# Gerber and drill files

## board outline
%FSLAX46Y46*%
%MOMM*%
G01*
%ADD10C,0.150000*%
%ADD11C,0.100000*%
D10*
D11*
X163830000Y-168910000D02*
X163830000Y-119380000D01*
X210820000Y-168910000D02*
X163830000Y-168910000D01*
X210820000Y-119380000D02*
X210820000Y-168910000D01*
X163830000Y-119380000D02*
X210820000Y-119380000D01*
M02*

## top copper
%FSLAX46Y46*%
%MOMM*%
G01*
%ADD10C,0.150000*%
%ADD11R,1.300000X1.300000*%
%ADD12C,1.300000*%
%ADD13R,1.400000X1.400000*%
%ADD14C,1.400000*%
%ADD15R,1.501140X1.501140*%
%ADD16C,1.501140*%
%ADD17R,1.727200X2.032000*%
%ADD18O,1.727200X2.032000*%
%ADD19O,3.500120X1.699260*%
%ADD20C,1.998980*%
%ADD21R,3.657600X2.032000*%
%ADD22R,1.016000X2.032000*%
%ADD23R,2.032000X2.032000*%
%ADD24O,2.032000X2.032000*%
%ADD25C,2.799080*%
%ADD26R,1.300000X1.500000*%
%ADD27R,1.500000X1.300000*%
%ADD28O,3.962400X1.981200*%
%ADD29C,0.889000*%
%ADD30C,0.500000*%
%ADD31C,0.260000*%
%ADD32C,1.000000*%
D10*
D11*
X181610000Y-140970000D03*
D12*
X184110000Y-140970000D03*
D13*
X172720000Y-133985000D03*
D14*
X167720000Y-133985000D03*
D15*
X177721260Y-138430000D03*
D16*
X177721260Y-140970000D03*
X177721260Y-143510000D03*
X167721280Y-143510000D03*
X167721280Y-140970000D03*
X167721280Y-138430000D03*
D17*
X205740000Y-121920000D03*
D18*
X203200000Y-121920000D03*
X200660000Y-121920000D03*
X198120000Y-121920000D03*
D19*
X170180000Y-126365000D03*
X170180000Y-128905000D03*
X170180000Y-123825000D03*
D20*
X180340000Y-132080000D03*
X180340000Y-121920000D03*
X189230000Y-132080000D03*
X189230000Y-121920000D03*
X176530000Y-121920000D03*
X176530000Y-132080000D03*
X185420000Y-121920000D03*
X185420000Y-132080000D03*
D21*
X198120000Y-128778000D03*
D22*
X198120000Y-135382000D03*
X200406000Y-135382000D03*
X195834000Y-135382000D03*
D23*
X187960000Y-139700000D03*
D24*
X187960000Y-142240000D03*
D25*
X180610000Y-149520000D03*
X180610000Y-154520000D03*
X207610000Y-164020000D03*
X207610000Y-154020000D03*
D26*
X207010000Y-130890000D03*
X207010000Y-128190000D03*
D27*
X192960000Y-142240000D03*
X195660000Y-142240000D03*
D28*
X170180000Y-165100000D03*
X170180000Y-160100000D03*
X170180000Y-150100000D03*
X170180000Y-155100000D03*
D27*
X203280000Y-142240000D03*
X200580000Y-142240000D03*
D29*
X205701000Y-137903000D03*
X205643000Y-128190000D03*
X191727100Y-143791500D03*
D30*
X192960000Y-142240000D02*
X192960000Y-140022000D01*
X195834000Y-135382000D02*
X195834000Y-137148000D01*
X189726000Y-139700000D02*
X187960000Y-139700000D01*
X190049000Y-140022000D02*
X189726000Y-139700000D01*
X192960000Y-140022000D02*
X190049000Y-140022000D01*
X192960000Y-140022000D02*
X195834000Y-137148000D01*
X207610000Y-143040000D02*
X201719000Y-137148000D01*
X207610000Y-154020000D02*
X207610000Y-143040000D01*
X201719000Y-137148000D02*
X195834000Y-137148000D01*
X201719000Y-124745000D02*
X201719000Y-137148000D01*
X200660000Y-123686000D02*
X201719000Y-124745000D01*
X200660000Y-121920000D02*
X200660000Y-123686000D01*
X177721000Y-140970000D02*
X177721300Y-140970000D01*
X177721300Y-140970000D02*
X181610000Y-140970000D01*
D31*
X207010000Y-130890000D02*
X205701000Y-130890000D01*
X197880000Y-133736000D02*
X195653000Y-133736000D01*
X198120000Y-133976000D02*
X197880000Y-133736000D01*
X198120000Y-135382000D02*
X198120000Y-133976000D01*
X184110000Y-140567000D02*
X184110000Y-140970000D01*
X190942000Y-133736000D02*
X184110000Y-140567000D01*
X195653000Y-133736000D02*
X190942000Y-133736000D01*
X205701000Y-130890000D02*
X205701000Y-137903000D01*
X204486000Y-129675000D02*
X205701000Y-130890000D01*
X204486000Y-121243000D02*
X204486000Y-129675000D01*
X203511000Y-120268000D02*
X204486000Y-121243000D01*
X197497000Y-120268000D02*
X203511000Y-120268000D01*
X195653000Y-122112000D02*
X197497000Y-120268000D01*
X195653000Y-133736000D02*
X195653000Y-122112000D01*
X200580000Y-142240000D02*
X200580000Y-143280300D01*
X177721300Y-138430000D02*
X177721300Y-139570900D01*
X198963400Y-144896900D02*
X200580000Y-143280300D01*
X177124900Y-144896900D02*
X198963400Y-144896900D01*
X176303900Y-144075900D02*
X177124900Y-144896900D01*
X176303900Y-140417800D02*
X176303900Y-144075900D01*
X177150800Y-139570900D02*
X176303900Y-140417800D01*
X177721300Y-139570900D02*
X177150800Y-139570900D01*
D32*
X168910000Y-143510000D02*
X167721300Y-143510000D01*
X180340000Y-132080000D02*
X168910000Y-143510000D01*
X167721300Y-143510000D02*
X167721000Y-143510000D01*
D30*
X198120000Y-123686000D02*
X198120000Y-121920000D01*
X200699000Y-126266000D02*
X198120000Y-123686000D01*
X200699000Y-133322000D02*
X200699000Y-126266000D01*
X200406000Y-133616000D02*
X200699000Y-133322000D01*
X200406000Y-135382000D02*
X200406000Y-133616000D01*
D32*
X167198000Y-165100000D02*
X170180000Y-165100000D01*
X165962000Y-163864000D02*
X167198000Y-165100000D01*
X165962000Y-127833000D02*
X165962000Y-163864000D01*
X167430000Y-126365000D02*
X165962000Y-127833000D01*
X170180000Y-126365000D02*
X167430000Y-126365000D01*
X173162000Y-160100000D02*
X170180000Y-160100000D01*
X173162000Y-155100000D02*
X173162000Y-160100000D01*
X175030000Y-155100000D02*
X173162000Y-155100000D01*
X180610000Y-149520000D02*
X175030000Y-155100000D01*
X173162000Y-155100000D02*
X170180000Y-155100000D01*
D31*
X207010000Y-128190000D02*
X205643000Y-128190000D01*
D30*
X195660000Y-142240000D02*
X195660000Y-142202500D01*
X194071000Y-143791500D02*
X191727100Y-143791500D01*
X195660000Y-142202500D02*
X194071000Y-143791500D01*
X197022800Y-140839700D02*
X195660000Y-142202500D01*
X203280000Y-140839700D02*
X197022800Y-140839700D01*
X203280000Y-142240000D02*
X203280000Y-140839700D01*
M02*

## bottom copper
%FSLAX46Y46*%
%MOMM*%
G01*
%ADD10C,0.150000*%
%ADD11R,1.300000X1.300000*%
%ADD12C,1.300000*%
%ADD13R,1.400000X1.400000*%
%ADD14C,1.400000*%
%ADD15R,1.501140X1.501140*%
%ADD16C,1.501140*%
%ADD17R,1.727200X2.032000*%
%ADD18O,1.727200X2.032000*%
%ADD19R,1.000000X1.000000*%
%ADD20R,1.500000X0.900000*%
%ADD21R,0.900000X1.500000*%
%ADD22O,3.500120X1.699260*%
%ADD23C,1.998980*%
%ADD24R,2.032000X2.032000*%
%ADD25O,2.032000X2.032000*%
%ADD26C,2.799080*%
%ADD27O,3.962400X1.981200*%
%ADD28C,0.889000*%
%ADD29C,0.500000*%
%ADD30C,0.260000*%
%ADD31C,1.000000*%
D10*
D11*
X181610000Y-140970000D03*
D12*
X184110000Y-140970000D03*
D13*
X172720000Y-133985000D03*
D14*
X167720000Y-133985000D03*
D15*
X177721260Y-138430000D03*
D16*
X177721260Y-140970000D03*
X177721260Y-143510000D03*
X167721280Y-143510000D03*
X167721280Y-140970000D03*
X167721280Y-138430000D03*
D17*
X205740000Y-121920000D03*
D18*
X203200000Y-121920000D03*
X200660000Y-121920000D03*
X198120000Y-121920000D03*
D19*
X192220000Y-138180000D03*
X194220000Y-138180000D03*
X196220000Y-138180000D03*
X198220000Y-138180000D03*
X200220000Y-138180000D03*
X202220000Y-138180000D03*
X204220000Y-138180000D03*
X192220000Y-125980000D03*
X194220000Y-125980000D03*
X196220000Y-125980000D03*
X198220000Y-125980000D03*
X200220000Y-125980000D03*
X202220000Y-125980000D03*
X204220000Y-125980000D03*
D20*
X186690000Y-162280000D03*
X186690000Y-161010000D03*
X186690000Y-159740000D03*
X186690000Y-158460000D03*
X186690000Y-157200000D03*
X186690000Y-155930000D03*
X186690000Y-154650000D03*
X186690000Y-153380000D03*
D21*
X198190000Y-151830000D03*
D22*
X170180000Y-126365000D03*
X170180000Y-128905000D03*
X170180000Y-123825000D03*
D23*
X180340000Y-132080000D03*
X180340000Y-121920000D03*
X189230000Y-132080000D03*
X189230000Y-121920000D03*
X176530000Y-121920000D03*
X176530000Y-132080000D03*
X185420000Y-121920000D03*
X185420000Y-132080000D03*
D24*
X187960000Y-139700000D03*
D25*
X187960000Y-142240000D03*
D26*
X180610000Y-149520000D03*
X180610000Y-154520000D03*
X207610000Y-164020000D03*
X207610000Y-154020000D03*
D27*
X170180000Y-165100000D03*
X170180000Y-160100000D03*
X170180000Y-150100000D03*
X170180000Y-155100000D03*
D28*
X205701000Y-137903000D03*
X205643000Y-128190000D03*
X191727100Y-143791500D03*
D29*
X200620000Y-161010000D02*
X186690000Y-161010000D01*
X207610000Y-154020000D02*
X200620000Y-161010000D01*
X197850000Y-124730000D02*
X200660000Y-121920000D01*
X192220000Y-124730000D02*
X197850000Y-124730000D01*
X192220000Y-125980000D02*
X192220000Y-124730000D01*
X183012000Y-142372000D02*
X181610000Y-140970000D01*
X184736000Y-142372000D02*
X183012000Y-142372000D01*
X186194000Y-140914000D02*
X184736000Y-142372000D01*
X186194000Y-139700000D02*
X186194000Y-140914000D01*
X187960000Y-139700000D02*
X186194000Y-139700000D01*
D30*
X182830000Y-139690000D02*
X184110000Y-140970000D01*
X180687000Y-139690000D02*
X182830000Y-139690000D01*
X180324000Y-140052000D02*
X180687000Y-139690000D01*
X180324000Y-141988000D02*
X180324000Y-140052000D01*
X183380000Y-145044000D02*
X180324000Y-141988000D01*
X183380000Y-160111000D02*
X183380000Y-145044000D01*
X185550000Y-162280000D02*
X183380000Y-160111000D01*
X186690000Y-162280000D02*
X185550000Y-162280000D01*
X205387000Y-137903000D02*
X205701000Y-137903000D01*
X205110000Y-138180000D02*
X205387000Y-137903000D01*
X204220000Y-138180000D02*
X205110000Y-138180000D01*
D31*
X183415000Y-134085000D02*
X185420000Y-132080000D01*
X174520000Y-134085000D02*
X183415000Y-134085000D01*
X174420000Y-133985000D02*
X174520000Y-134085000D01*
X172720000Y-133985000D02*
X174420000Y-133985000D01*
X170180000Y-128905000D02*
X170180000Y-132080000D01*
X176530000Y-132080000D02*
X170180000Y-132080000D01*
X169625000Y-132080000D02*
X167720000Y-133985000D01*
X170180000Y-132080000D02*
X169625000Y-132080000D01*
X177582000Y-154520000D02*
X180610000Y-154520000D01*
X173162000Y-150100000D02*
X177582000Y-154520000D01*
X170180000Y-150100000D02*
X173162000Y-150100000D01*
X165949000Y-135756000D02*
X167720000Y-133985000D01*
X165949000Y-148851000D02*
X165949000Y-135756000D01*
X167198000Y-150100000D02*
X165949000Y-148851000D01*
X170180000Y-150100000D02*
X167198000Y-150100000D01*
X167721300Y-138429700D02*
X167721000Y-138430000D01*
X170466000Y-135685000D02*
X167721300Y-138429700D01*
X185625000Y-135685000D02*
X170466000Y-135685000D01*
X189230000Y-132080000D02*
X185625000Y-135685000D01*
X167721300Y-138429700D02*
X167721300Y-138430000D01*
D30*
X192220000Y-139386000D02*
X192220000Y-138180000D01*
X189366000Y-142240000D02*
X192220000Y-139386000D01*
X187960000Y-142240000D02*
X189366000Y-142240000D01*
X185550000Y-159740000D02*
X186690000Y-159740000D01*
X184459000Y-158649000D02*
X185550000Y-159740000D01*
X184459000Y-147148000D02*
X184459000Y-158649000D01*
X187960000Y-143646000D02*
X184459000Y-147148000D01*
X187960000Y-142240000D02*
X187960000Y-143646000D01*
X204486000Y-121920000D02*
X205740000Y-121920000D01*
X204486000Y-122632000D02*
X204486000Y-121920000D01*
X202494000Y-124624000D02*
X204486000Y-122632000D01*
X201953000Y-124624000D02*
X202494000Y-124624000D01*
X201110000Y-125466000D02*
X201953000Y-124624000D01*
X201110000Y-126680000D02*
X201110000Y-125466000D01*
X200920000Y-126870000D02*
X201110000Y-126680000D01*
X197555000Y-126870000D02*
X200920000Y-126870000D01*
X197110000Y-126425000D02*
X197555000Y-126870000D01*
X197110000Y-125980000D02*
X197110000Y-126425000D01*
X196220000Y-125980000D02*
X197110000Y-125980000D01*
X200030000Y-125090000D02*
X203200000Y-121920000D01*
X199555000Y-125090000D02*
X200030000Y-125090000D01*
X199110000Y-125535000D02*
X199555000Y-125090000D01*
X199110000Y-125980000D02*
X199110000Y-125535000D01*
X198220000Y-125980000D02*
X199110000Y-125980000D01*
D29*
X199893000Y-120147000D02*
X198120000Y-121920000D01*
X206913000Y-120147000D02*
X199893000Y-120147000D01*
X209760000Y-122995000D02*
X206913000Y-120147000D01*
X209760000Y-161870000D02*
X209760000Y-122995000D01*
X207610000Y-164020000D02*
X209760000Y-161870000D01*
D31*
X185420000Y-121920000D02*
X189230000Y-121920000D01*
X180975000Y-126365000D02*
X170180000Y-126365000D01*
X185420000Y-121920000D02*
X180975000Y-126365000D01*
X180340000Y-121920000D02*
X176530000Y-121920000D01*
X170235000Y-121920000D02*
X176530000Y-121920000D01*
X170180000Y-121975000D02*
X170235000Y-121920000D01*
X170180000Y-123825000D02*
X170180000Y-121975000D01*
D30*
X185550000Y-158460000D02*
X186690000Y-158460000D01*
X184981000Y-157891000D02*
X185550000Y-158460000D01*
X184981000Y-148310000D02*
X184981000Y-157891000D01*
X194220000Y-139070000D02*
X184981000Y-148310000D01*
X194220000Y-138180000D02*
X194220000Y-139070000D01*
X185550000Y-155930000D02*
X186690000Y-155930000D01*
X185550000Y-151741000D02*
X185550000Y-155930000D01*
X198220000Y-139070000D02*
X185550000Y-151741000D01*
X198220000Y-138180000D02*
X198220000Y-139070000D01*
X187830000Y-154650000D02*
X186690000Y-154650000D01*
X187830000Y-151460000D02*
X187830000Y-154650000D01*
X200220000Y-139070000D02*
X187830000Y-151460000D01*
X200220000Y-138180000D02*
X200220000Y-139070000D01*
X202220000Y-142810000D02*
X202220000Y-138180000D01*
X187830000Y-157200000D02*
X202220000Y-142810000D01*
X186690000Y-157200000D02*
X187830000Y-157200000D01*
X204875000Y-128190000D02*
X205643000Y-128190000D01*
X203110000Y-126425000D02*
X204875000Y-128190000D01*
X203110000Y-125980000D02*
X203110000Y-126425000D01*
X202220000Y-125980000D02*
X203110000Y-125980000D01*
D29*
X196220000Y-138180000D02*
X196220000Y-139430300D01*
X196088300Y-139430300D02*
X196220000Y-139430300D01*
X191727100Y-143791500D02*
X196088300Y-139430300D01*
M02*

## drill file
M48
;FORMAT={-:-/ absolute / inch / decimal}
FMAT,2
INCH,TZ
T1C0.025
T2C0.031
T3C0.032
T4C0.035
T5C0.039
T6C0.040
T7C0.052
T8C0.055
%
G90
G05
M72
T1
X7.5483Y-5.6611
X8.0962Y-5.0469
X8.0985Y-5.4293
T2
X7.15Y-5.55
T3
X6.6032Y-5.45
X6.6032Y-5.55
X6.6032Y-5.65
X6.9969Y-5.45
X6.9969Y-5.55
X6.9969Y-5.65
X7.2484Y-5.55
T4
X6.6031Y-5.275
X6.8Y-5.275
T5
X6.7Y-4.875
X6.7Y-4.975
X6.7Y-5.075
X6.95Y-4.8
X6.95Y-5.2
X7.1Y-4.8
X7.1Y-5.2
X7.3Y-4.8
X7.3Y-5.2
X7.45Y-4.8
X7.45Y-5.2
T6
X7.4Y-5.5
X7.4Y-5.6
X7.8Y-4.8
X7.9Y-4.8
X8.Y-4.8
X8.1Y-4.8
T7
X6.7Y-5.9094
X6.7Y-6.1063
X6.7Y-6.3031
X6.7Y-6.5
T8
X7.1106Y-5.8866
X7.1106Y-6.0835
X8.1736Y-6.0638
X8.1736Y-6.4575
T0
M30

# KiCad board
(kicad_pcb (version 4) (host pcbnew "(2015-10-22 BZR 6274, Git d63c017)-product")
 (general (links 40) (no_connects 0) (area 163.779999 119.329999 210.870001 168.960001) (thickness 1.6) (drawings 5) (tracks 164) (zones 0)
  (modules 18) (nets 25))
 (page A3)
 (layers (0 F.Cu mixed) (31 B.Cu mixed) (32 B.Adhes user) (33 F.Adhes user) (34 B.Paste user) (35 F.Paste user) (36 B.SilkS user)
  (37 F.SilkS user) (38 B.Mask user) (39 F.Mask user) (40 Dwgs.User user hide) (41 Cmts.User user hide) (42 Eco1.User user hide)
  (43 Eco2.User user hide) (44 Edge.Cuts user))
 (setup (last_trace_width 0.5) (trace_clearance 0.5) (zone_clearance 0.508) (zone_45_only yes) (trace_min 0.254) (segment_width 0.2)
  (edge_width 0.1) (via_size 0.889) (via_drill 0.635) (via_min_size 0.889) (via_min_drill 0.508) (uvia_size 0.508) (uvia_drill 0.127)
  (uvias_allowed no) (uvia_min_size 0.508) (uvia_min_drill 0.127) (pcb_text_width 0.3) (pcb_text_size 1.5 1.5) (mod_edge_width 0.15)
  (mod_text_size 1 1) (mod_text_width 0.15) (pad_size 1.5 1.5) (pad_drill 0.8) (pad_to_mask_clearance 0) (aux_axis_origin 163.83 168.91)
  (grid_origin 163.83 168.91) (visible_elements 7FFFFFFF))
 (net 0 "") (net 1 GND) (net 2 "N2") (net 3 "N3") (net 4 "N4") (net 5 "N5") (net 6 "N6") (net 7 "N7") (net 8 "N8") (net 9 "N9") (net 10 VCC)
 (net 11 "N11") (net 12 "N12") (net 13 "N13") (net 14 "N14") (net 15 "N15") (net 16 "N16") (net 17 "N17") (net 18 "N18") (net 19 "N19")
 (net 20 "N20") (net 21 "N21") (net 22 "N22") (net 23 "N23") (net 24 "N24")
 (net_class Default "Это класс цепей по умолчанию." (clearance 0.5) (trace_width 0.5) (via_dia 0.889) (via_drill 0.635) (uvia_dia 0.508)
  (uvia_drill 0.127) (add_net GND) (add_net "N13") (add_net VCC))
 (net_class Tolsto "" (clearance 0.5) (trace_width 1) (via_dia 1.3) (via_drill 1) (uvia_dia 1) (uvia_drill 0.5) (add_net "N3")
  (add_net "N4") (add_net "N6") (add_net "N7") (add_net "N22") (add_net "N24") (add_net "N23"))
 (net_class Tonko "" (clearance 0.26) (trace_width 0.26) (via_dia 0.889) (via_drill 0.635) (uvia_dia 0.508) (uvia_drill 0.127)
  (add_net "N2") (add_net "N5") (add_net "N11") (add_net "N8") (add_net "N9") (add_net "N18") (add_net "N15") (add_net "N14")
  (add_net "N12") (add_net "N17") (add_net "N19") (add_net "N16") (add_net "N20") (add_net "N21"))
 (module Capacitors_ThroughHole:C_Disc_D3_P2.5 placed (layer F.Cu) (at 181.61 140.97)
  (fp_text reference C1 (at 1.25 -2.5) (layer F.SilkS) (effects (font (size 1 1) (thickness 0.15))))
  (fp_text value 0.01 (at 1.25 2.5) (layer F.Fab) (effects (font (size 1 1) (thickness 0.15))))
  (pad 1 thru_hole rect (at 0 0) (size 1.3 1.3) (drill 0.8) (layers *.Cu *.Mask F.SilkS) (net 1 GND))
  (pad 2 thru_hole circle (at 2.5 0) (size 1.3 1.3) (drill 0.8001) (layers *.Cu *.Mask F.SilkS) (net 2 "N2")))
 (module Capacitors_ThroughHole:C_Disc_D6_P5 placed (layer F.Cu) (at 172.72 133.985 180)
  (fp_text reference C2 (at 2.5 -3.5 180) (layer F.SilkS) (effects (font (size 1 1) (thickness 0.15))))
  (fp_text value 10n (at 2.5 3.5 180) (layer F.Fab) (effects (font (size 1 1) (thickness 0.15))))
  (pad 1 thru_hole rect (at 0 0 180) (size 1.4 1.4) (drill 0.9) (layers *.Cu *.Mask F.SilkS) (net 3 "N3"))
  (pad 2 thru_hole circle (at 5 0 180) (size 1.4 1.4) (drill 0.9) (layers *.Cu *.Mask F.SilkS) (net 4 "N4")))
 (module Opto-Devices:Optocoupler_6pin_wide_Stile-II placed (layer B.Cu) (at 172.72 140.97 270)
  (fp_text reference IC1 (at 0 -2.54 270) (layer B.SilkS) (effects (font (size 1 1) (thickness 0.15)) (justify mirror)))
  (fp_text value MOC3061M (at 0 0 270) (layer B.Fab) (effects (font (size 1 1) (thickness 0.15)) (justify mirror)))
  (pad 1 thru_hole rect (at -2.54 -5.00126 270) (size 1.50114 1.50114) (drill 0.8001) (layers *.Cu *.Mask B.SilkS) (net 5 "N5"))
  (pad 2 thru_hole circle (at 0 -5.00126 270) (size 1.50114 1.50114) (drill 0.8001) (layers *.Cu *.Mask B.SilkS) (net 1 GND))
  (pad 3 thru_hole circle (at 2.54 -5.00126 270) (size 1.50114 1.50114) (drill 0.8001) (layers *.Cu *.Mask B.SilkS))
  (pad 4 thru_hole circle (at 2.54 4.99872 270) (size 1.50114 1.50114) (drill 0.8001) (layers *.Cu *.Mask B.SilkS) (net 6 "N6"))
  (pad 5 thru_hole circle (at 0 4.99872 270) (size 1.50114 1.50114) (drill 0.8001) (layers *.Cu *.Mask B.SilkS))
  (pad 6 thru_hole circle (at -2.54 4.99872 270) (size 1.50114 1.50114) (drill 0.8001) (layers *.Cu *.Mask B.SilkS) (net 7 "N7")))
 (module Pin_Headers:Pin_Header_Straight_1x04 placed (layer F.Cu) (at 205.74 121.92 270)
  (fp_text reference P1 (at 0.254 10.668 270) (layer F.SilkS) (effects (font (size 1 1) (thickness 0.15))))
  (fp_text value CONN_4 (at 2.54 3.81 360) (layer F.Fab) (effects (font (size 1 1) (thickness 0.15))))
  (pad 1 thru_hole rect (at 0 0 270) (size 2.032 1.7272) (drill 1.016) (layers *.Cu *.Mask F.SilkS) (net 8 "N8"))
  (pad 2 thru_hole oval (at 0 2.54 270) (size 2.032 1.7272) (drill 1.016) (layers *.Cu *.Mask F.SilkS) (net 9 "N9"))
  (pad 3 thru_hole oval (at 0 5.08 270) (size 2.032 1.7272) (drill 1.016) (layers *.Cu *.Mask F.SilkS) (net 1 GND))
  (pad 4 thru_hole oval (at 0 7.62 270) (size 2.032 1.7272) (drill 1.016) (layers *.Cu *.Mask F.SilkS) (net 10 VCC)))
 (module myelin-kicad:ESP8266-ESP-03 (layer B.Cu) (at 198.12 132.08 90)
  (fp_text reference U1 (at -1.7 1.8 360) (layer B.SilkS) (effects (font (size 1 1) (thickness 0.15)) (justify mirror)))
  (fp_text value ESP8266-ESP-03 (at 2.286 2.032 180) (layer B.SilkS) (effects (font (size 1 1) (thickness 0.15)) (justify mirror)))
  (pad 14 smd rect (at -6.1 -5.9 90) (size 1 1) (layers B.Cu B.Paste B.Mask) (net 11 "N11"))
  (pad 13 smd rect (at -6.1 -3.9 90) (size 1 1) (layers B.Cu B.Paste B.Mask) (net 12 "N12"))
  (pad 12 smd rect (at -6.1 -1.9 90) (size 1 1) (layers B.Cu B.Paste B.Mask) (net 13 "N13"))
  (pad 11 smd rect (at -6.1 0.1 90) (size 1 1) (layers B.Cu B.Paste B.Mask) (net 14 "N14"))
  (pad 10 smd rect (at -6.1 2.1 90) (size 1 1) (layers B.Cu B.Paste B.Mask) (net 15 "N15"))
  (pad 9 smd rect (at -6.1 4.1 90) (size 1 1) (layers B.Cu B.Paste B.Mask) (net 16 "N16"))
  (pad 8 smd rect (at -6.1 6.1 90) (size 1 1) (layers B.Cu B.Paste B.Mask) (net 2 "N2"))
  (pad 1 smd rect (at 6.1 -5.9 90) (size 1 1) (layers B.Cu B.Paste B.Mask) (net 1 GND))
  (pad 2 smd rect (at 6.1 -3.9 90) (size 1 1) (layers B.Cu B.Paste B.Mask))
  (pad 3 smd rect (at 6.1 -1.9 90) (size 1 1) (layers B.Cu B.Paste B.Mask) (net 8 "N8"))
  (pad 4 smd rect (at 6.1 0.1 90) (size 1 1) (layers B.Cu B.Paste B.Mask) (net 9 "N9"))
  (pad 5 smd rect (at 6.1 2.1 90) (size 1 1) (layers B.Cu B.Paste B.Mask) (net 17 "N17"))
  (pad 6 smd rect (at 6.1 4.1 90) (size 1 1) (layers B.Cu B.Paste B.Mask) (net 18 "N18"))
  (pad 7 smd rect (at 6.1 6.1 90) (size 1 1) (layers B.Cu B.Paste B.Mask) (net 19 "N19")))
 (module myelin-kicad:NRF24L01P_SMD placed (layer B.Cu) (at 186.69 163.83)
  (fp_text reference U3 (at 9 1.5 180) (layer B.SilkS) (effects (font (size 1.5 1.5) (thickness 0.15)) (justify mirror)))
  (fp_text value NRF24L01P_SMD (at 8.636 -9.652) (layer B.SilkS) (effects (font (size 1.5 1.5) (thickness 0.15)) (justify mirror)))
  (pad 1 smd rect (at 0 -1.55) (size 1.5 0.9) (layers B.Cu B.Paste B.Mask) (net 2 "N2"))
  (pad 2 smd rect (at 0 -2.82) (size 1.5 0.9) (layers B.Cu B.Paste B.Mask) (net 1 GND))
  (pad 3 smd rect (at 0 -4.09) (size 1.5 0.9) (layers B.Cu B.Paste B.Mask) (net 11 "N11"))
  (pad 4 smd rect (at 0 -5.37) (size 1.5 0.9) (layers B.Cu B.Paste B.Mask) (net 12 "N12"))
  (pad 5 smd rect (at 0 -6.63) (size 1.5 0.9) (layers B.Cu B.Paste B.Mask) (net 16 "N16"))
  (pad 6 smd rect (at 0 -7.9) (size 1.5 0.9) (layers B.Cu B.Paste B.Mask) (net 14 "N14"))
  (pad 7 smd rect (at 0 -9.18) (size 1.5 0.9) (layers B.Cu B.Paste B.Mask) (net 15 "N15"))
  (pad 8 smd rect (at 0 -10.45) (size 1.5 0.9) (layers B.Cu B.Paste B.Mask) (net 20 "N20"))
  (pad 9 smd rect (at 11.5 -12) (size 0.9 1.5) (layers B.Cu B.Paste B.Mask) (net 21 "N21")))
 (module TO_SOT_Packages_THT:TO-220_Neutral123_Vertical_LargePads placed (layer F.Cu) (at 170.18 126.365 90)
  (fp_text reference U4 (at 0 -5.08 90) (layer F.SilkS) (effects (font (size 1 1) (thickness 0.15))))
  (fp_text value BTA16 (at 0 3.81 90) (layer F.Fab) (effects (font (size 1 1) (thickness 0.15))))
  (pad 2 thru_hole oval (at 0 0 180) (size 3.50012 1.69926) (drill 1.00076) (layers *.Cu *.Mask F.SilkS) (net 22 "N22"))
  (pad 1 thru_hole oval (at -2.54 0 180) (size 3.50012 1.69926) (drill 1.00076) (layers *.Cu *.Mask F.SilkS) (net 4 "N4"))
  (pad 3 thru_hole oval (at 2.54 0 180) (size 3.50012 1.69926) (drill 1.00076) (layers *.Cu *.Mask F.SilkS) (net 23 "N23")))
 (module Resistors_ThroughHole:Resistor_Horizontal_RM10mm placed (layer F.Cu) (at 180.34 127 90)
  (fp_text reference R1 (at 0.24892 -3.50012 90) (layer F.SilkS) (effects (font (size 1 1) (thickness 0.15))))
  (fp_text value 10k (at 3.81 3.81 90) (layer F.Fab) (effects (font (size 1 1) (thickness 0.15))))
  (pad 1 thru_hole circle (at -5.08 0 90) (size 1.99898 1.99898) (drill 1.00076) (layers *.Cu *.SilkS *.Mask) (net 6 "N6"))
  (pad 2 thru_hole circle (at 5.08 0 90) (size 1.99898 1.99898) (drill 1.00076) (layers *.Cu *.SilkS *.Mask) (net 23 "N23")))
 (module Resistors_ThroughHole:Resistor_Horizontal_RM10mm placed (layer F.Cu) (at 189.23 127 90)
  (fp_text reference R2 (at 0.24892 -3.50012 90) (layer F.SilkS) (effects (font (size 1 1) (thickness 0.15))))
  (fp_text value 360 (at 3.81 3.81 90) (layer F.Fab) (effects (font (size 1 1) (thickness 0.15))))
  (pad 1 thru_hole circle (at -5.08 0 90) (size 1.99898 1.99898) (drill 1.00076) (layers *.Cu *.SilkS *.Mask) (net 7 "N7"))
  (pad 2 thru_hole circle (at 5.08 0 90) (size 1.99898 1.99898) (drill 1.00076) (layers *.Cu *.SilkS *.Mask) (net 22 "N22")))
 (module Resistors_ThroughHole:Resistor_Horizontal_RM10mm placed (layer F.Cu) (at 176.53 127 270)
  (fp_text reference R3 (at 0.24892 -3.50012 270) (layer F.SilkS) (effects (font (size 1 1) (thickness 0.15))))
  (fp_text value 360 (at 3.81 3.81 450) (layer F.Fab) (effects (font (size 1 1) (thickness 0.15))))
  (pad 1 thru_hole circle (at -5.08 0 270) (size 1.99898 1.99898) (drill 1.00076) (layers *.Cu *.SilkS *.Mask) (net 23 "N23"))
  (pad 2 thru_hole circle (at 5.08 0 270) (size 1.99898 1.99898) (drill 1.00076) (layers *.Cu *.SilkS *.Mask) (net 4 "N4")))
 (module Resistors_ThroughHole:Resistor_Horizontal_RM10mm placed (layer F.Cu) (at 185.42 127 270)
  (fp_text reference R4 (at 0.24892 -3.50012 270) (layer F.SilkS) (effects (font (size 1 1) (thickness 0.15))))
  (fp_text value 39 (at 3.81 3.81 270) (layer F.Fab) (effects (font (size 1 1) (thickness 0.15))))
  (pad 1 thru_hole circle (at -5.08 0 270) (size 1.99898 1.99898) (drill 1.00076) (layers *.Cu *.SilkS *.Mask) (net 22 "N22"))
  (pad 2 thru_hole circle (at 5.08 0 270) (size 1.99898 1.99898) (drill 1.00076) (layers *.Cu *.SilkS *.Mask) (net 3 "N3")))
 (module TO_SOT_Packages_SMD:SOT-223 (layer F.Cu) (at 198.12 132.08)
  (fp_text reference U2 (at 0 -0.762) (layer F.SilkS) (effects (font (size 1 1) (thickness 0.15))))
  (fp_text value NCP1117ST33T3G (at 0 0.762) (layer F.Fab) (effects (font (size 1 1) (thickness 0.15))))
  (pad 4 smd rect (at 0 -3.302) (size 3.6576 2.032) (layers F.Cu F.Paste F.Mask))
  (pad 2 smd rect (at 0 3.302) (size 1.016 2.032) (layers F.Cu F.Paste F.Mask) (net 2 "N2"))
  (pad 3 smd rect (at 2.286 3.302) (size 1.016 2.032) (layers F.Cu F.Paste F.Mask) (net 10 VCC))
  (pad 1 smd rect (at -2.286 3.302) (size 1.016 2.032) (layers F.Cu F.Paste F.Mask) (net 1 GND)))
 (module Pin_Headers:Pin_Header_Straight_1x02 (layer F.Cu) (at 187.96 139.7)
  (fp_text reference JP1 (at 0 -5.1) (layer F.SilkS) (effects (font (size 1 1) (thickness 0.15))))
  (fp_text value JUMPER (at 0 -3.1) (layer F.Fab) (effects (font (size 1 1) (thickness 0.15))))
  (pad 1 thru_hole rect (at 0 0) (size 2.032 2.032) (drill 1.016) (layers *.Cu *.Mask F.SilkS) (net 1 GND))
  (pad 2 thru_hole oval (at 0 2.54) (size 2.032 2.032) (drill 1.016) (layers *.Cu *.Mask F.SilkS) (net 11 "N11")))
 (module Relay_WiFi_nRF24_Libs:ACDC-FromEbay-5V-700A (layer F.Cu) (at 181.61 160.02)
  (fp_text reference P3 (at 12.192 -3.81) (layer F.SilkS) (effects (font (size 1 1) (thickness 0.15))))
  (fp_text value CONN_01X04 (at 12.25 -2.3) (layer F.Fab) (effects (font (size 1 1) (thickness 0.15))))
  (pad 1 thru_hole circle (at -1 -10.5) (size 2.79908 2.79908) (drill 1.39954) (layers *.Cu *.Mask F.SilkS) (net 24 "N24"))
  (pad 2 thru_hole circle (at -1 -5.5) (size 2.79908 2.79908) (drill 1.39954) (layers *.Cu *.Mask F.SilkS) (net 4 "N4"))
  (pad 3 thru_hole circle (at 26 4) (size 2.79908 2.79908) (drill 1.39954) (layers *.Cu *.Mask F.SilkS) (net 10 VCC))
  (pad 4 thru_hole circle (at 26 -6) (size 2.79908 2.79908) (drill 1.39954) (layers *.Cu *.Mask F.SilkS) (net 1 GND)))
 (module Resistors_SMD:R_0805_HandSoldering (layer F.Cu) (at 207.01 129.54 90)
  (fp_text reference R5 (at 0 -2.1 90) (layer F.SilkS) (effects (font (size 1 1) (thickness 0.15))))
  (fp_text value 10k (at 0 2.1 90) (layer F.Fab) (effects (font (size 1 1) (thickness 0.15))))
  (pad 1 smd rect (at -1.35 0 90) (size 1.5 1.3) (layers F.Cu F.Paste F.Mask) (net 2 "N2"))
  (pad 2 smd rect (at 1.35 0 90) (size 1.5 1.3) (layers F.Cu F.Paste F.Mask) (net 18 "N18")))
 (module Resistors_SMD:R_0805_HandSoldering (layer F.Cu) (at 194.31 142.24)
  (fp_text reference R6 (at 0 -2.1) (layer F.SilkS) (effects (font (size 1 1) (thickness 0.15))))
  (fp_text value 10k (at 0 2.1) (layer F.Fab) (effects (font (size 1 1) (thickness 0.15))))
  (pad 1 smd rect (at -1.35 0) (size 1.5 1.3) (layers F.Cu F.Paste F.Mask) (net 1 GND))
  (pad 2 smd rect (at 1.35 0) (size 1.5 1.3) (layers F.Cu F.Paste F.Mask) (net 13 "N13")))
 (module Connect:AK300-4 (layer F.Cu) (at 170.18 165.1 90)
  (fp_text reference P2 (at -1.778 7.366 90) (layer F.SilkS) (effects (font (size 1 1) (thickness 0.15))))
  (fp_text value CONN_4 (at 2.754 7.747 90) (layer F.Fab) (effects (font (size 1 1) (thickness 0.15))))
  (pad 1 thru_hole oval (at 0 0 90) (size 1.9812 3.9624) (drill 1.3208) (layers *.Cu F.Paste F.SilkS F.Mask) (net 22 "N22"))
  (pad 2 thru_hole oval (at 5 0 90) (size 1.9812 3.9624) (drill 1.3208) (layers *.Cu F.Paste F.SilkS F.Mask) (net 24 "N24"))
  (pad 4 thru_hole oval (at 15 0 90) (size 1.9812 3.9624) (drill 1.3208) (layers *.Cu F.Paste F.SilkS F.Mask) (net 4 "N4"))
  (pad 3 thru_hole oval (at 10 0 90) (size 1.9812 3.9624) (drill 1.3208) (layers *.Cu *.Mask F.SilkS) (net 24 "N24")))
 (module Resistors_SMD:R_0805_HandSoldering (layer F.Cu) (at 201.93 142.24 180)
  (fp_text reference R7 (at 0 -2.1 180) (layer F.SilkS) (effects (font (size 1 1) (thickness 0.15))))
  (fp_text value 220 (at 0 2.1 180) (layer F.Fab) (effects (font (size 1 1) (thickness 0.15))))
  (pad 1 smd rect (at -1.35 0 180) (size 1.5 1.3) (layers F.Cu F.Paste F.Mask) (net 13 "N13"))
  (pad 2 smd rect (at 1.35 0 180) (size 1.5 1.3) (layers F.Cu F.Paste F.Mask) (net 5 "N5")))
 (gr_line (start 163.83 168.91) (end 163.83 119.38) (angle 90) (layer Edge.Cuts) (width 0.1))
 (gr_line (start 210.82 168.91) (end 163.83 168.91) (angle 90) (layer Edge.Cuts) (width 0.1))
 (gr_line (start 210.82 119.38) (end 210.82 168.91) (angle 90) (layer Edge.Cuts) (width 0.1))
 (gr_line (start 163.83 119.38) (end 210.82 119.38) (angle 90) (layer Edge.Cuts) (width 0.1))
 (segment (start 200.62 161.01) (end 186.69 161.01) (width 0.5) (layer B.Cu) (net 1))
 (segment (start 207.61 154.02) (end 200.62 161.01) (width 0.5) (layer B.Cu) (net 1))
 (segment (start 197.85 124.73) (end 200.66 121.92) (width 0.5) (layer B.Cu) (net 1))
 (segment (start 192.22 124.73) (end 197.85 124.73) (width 0.5) (layer B.Cu) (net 1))
 (segment (start 192.22 125.98) (end 192.22 124.73) (width 0.5) (layer B.Cu) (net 1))
 (segment (start 183.012 142.372) (end 181.61 140.97) (width 0.5) (layer B.Cu) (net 1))
 (segment (start 184.736 142.372) (end 183.012 142.372) (width 0.5) (layer B.Cu) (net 1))
 (segment (start 186.194 140.914) (end 184.736 142.372) (width 0.5) (layer B.Cu) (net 1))
 (segment (start 186.194 139.7) (end 186.194 140.914) (width 0.5) (layer B.Cu) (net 1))
 (segment (start 187.96 139.7) (end 186.194 139.7) (width 0.5) (layer B.Cu) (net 1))
 (segment (start 192.96 142.24) (end 192.96 140.022) (width 0.5) (layer F.Cu) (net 1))
 (segment (start 195.834 135.382) (end 195.834 137.148) (width 0.5) (layer F.Cu) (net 1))
 (segment (start 189.726 139.7) (end 187.96 139.7) (width 0.5) (layer F.Cu) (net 1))
 (segment (start 190.049 140.022) (end 189.726 139.7) (width 0.5) (layer F.Cu) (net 1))
 (segment (start 192.96 140.022) (end 190.049 140.022) (width 0.5) (layer F.Cu) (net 1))
 (segment (start 192.96 140.022) (end 195.834 137.148) (width 0.5) (layer F.Cu) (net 1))
 (segment (start 207.61 143.04) (end 201.719 137.148) (width 0.5) (layer F.Cu) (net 1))
 (segment (start 207.61 154.02) (end 207.61 143.04) (width 0.5) (layer F.Cu) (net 1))
 (segment (start 201.719 137.148) (end 195.834 137.148) (width 0.5) (layer F.Cu) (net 1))
 (segment (start 201.719 124.745) (end 201.719 137.148) (width 0.5) (layer F.Cu) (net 1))
 (segment (start 200.66 123.686) (end 201.719 124.745) (width 0.5) (layer F.Cu) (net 1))
 (segment (start 200.66 121.92) (end 200.66 123.686) (width 0.5) (layer F.Cu) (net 1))
 (segment (start 177.721 140.97) (end 177.7213 140.97) (width 0.5) (layer F.Cu) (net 1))
 (segment (start 177.7213 140.97) (end 181.61 140.97) (width 0.5) (layer F.Cu) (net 1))
 (via (at 205.701 137.903) (size 0.889) (layers F.Cu B.Cu) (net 2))
 (segment (start 182.83 139.69) (end 184.11 140.97) (width 0.26) (layer B.Cu) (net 2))
 (segment (start 180.687 139.69) (end 182.83 139.69) (width 0.26) (layer B.Cu) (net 2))
 (segment (start 180.324 140.052) (end 180.687 139.69) (width 0.26) (layer B.Cu) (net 2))
 (segment (start 180.324 141.988) (end 180.324 140.052) (width 0.26) (layer B.Cu) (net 2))
 (segment (start 183.38 145.044) (end 180.324 141.988) (width 0.26) (layer B.Cu) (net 2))
 (segment (start 183.38 160.111) (end 183.38 145.044) (width 0.26) (layer B.Cu) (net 2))
 (segment (start 185.55 162.28) (end 183.38 160.111) (width 0.26) (layer B.Cu) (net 2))
 (segment (start 186.69 162.28) (end 185.55 162.28) (width 0.26) (layer B.Cu) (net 2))
 (segment (start 207.01 130.89) (end 205.701 130.89) (width 0.26) (layer F.Cu) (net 2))
 (segment (start 197.88 133.736) (end 195.653 133.736) (width 0.26) (layer F.Cu) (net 2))
 (segment (start 198.12 133.976) (end 197.88 133.736) (width 0.26) (layer F.Cu) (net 2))
 (segment (start 198.12 135.382) (end 198.12 133.976) (width 0.26) (layer F.Cu) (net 2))
 (segment (start 184.11 140.567) (end 184.11 140.97) (width 0.26) (layer F.Cu) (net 2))
 (segment (start 190.942 133.736) (end 184.11 140.567) (width 0.26) (layer F.Cu) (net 2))
 (segment (start 195.653 133.736) (end 190.942 133.736) (width 0.26) (layer F.Cu) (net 2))
 (segment (start 205.701 130.89) (end 205.701 137.903) (width 0.26) (layer F.Cu) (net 2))
 (segment (start 204.486 129.675) (end 205.701 130.89) (width 0.26) (layer F.Cu) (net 2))
 (segment (start 204.486 121.243) (end 204.486 129.675) (width 0.26) (layer F.Cu) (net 2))
 (segment (start 203.511 120.268) (end 204.486 121.243) (width 0.26) (layer F.Cu) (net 2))
 (segment (start 197.497 120.268) (end 203.511 120.268) (width 0.26) (layer F.Cu) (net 2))
 (segment (start 195.653 122.112) (end 197.497 120.268) (width 0.26) (layer F.Cu) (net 2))
 (segment (start 195.653 133.736) (end 195.653 122.112) (width 0.26) (layer F.Cu) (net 2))
 (segment (start 205.387 137.903) (end 205.701 137.903) (width 0.26) (layer B.Cu) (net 2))
 (segment (start 205.11 138.18) (end 205.387 137.903) (width 0.26) (layer B.Cu) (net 2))
 (segment (start 204.22 138.18) (end 205.11 138.18) (width 0.26) (layer B.Cu) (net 2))
 (segment (start 183.415 134.085) (end 185.42 132.08) (width 1) (layer B.Cu) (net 3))
 (segment (start 174.52 134.085) (end 183.415 134.085) (width 1) (layer B.Cu) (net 3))
 (segment (start 174.42 133.985) (end 174.52 134.085) (width 1) (layer B.Cu) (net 3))
 (segment (start 172.72 133.985) (end 174.42 133.985) (width 1) (layer B.Cu) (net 3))
 (segment (start 170.18 128.905) (end 170.18 132.08) (width 1) (layer B.Cu) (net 4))
 (segment (start 176.53 132.08) (end 170.18 132.08) (width 1) (layer B.Cu) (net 4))
 (segment (start 169.625 132.08) (end 167.72 133.985) (width 1) (layer B.Cu) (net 4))
 (segment (start 170.18 132.08) (end 169.625 132.08) (width 1) (layer B.Cu) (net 4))
 (segment (start 177.582 154.52) (end 180.61 154.52) (width 1) (layer B.Cu) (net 4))
 (segment (start 173.162 150.1) (end 177.582 154.52) (width 1) (layer B.Cu) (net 4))
 (segment (start 170.18 150.1) (end 173.162 150.1) (width 1) (layer B.Cu) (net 4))
 (segment (start 165.949 135.756) (end 167.72 133.985) (width 1) (layer B.Cu) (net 4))
 (segment (start 165.949 148.851) (end 165.949 135.756) (width 1) (layer B.Cu) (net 4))
 (segment (start 167.198 150.1) (end 165.949 148.851) (width 1) (layer B.Cu) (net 4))
 (segment (start 170.18 150.1) (end 167.198 150.1) (width 1) (layer B.Cu) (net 4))
 (segment (start 200.58 142.24) (end 200.58 143.2803) (width 0.26) (layer F.Cu) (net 5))
 (segment (start 177.7213 138.43) (end 177.7213 139.5709) (width 0.26) (layer F.Cu) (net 5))
 (segment (start 198.9634 144.8969) (end 200.58 143.2803) (width 0.26) (layer F.Cu) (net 5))
 (segment (start 177.1249 144.8969) (end 198.9634 144.8969) (width 0.26) (layer F.Cu) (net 5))
 (segment (start 176.3039 144.0759) (end 177.1249 144.8969) (width 0.26) (layer F.Cu) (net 5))
 (segment (start 176.3039 140.4178) (end 176.3039 144.0759) (width 0.26) (layer F.Cu) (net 5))
 (segment (start 177.1508 139.5709) (end 176.3039 140.4178) (width 0.26) (layer F.Cu) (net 5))
 (segment (start 177.7213 139.5709) (end 177.1508 139.5709) (width 0.26) (layer F.Cu) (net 5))
 (segment (start 168.91 143.51) (end 167.7213 143.51) (width 1) (layer F.Cu) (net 6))
 (segment (start 180.34 132.08) (end 168.91 143.51) (width 1) (layer F.Cu) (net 6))
 (segment (start 167.7213 143.51) (end 167.721 143.51) (width 1) (layer F.Cu) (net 6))
 (segment (start 167.7213 138.4297) (end 167.721 138.43) (width 1) (layer B.Cu) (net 7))
 (segment (start 170.466 135.685) (end 167.7213 138.4297) (width 1) (layer B.Cu) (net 7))
 (segment (start 185.625 135.685) (end 170.466 135.685) (width 1) (layer B.Cu) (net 7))
 (segment (start 189.23 132.08) (end 185.625 135.685) (width 1) (layer B.Cu) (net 7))
 (segment (start 167.7213 138.4297) (end 167.7213 138.43) (width 1) (layer B.Cu) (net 7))
 (segment (start 192.22 139.386) (end 192.22 138.18) (width 0.26) (layer B.Cu) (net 11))
 (segment (start 189.366 142.24) (end 192.22 139.386) (width 0.26) (layer B.Cu) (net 11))
 (segment (start 187.96 142.24) (end 189.366 142.24) (width 0.26) (layer B.Cu) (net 11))
 (segment (start 185.55 159.74) (end 186.69 159.74) (width 0.26) (layer B.Cu) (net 11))
 (segment (start 184.459 158.649) (end 185.55 159.74) (width 0.26) (layer B.Cu) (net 11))
 (segment (start 184.459 147.148) (end 184.459 158.649) (width 0.26) (layer B.Cu) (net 11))
 (segment (start 187.96 143.646) (end 184.459 147.148) (width 0.26) (layer B.Cu) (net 11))
 (segment (start 187.96 142.24) (end 187.96 143.646) (width 0.26) (layer B.Cu) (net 11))
 (segment (start 204.486 121.92) (end 205.74 121.92) (width 0.26) (layer B.Cu) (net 8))
 (segment (start 204.486 122.632) (end 204.486 121.92) (width 0.26) (layer B.Cu) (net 8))
 (segment (start 202.494 124.624) (end 204.486 122.632) (width 0.26) (layer B.Cu) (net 8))
 (segment (start 201.953 124.624) (end 202.494 124.624) (width 0.26) (layer B.Cu) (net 8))
 (segment (start 201.11 125.466) (end 201.953 124.624) (width 0.26) (layer B.Cu) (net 8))
 (segment (start 201.11 126.68) (end 201.11 125.466) (width 0.26) (layer B.Cu) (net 8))
 (segment (start 200.92 126.87) (end 201.11 126.68) (width 0.26) (layer B.Cu) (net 8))
 (segment (start 197.555 126.87) (end 200.92 126.87) (width 0.26) (layer B.Cu) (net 8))
 (segment (start 197.11 126.425) (end 197.555 126.87) (width 0.26) (layer B.Cu) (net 8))
 (segment (start 197.11 125.98) (end 197.11 126.425) (width 0.26) (layer B.Cu) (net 8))
 (segment (start 196.22 125.98) (end 197.11 125.98) (width 0.26) (layer B.Cu) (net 8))
 (segment (start 200.03 125.09) (end 203.2 121.92) (width 0.26) (layer B.Cu) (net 9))
 (segment (start 199.555 125.09) (end 200.03 125.09) (width 0.26) (layer B.Cu) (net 9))
 (segment (start 199.11 125.535) (end 199.555 125.09) (width 0.26) (layer B.Cu) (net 9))
 (segment (start 199.11 125.98) (end 199.11 125.535) (width 0.26) (layer B.Cu) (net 9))
 (segment (start 198.22 125.98) (end 199.11 125.98) (width 0.26) (layer B.Cu) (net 9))
 (segment (start 199.893 120.147) (end 198.12 121.92) (width 0.5) (layer B.Cu) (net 10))
 (segment (start 206.913 120.147) (end 199.893 120.147) (width 0.5) (layer B.Cu) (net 10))
 (segment (start 209.76 122.995) (end 206.913 120.147) (width 0.5) (layer B.Cu) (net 10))
 (segment (start 209.76 161.87) (end 209.76 122.995) (width 0.5) (layer B.Cu) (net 10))
 (segment (start 207.61 164.02) (end 209.76 161.87) (width 0.5) (layer B.Cu) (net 10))
 (segment (start 198.12 123.686) (end 198.12 121.92) (width 0.5) (layer F.Cu) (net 10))
 (segment (start 200.699 126.266) (end 198.12 123.686) (width 0.5) (layer F.Cu) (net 10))
 (segment (start 200.699 133.322) (end 200.699 126.266) (width 0.5) (layer F.Cu) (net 10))
 (segment (start 200.406 133.616) (end 200.699 133.322) (width 0.5) (layer F.Cu) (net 10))
 (segment (start 200.406 135.382) (end 200.406 133.616) (width 0.5) (layer F.Cu) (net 10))
 (segment (start 185.42 121.92) (end 189.23 121.92) (width 1) (layer B.Cu) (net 22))
 (segment (start 180.975 126.365) (end 170.18 126.365) (width 1) (layer B.Cu) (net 22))
 (segment (start 185.42 121.92) (end 180.975 126.365) (width 1) (layer B.Cu) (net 22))
 (segment (start 167.198 165.1) (end 170.18 165.1) (width 1) (layer F.Cu) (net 22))
 (segment (start 165.962 163.864) (end 167.198 165.1) (width 1) (layer F.Cu) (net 22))
 (segment (start 165.962 127.833) (end 165.962 163.864) (width 1) (layer F.Cu) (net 22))
 (segment (start 167.43 126.365) (end 165.962 127.833) (width 1) (layer F.Cu) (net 22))
 (segment (start 170.18 126.365) (end 167.43 126.365) (width 1) (layer F.Cu) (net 22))
 (segment (start 173.162 160.1) (end 170.18 160.1) (width 1) (layer F.Cu) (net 24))
 (segment (start 173.162 155.1) (end 173.162 160.1) (width 1) (layer F.Cu) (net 24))
 (segment (start 175.03 155.1) (end 173.162 155.1) (width 1) (layer F.Cu) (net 24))
 (segment (start 180.61 149.52) (end 175.03 155.1) (width 1) (layer F.Cu) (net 24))
 (segment (start 173.162 155.1) (end 170.18 155.1) (width 1) (layer F.Cu) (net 24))
 (segment (start 180.34 121.92) (end 176.53 121.92) (width 1) (layer B.Cu) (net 23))
 (segment (start 170.235 121.92) (end 176.53 121.92) (width 1) (layer B.Cu) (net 23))
 (segment (start 170.18 121.975) (end 170.235 121.92) (width 1) (layer B.Cu) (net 23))
 (segment (start 170.18 123.825) (end 170.18 121.975) (width 1) (layer B.Cu) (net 23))
 (segment (start 185.55 158.46) (end 186.69 158.46) (width 0.26) (layer B.Cu) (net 12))
 (segment (start 184.981 157.891) (end 185.55 158.46) (width 0.26) (layer B.Cu) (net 12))
 (segment (start 184.981 148.31) (end 184.981 157.891) (width 0.26) (layer B.Cu) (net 12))
 (segment (start 194.22 139.07) (end 184.981 148.31) (width 0.26) (layer B.Cu) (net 12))
 (segment (start 194.22 138.18) (end 194.22 139.07) (width 0.26) (layer B.Cu) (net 12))
 (segment (start 185.55 155.93) (end 186.69 155.93) (width 0.26) (layer B.Cu) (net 14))
 (segment (start 185.55 151.741) (end 185.55 155.93) (width 0.26) (layer B.Cu) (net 14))
 (segment (start 198.22 139.07) (end 185.55 151.741) (width 0.26) (layer B.Cu) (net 14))
 (segment (start 198.22 138.18) (end 198.22 139.07) (width 0.26) (layer B.Cu) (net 14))
 (segment (start 187.83 154.65) (end 186.69 154.65) (width 0.26) (layer B.Cu) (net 15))
 (segment (start 187.83 151.46) (end 187.83 154.65) (width 0.26) (layer B.Cu) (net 15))
 (segment (start 200.22 139.07) (end 187.83 151.46) (width 0.26) (layer B.Cu) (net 15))
 (segment (start 200.22 138.18) (end 200.22 139.07) (width 0.26) (layer B.Cu) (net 15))
 (segment (start 202.22 142.81) (end 202.22 138.18) (width 0.26) (layer B.Cu) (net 16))
 (segment (start 187.83 157.2) (end 202.22 142.81) (width 0.26) (layer B.Cu) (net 16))
 (segment (start 186.69 157.2) (end 187.83 157.2) (width 0.26) (layer B.Cu) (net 16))
 (via (at 205.643 128.19) (size 0.889) (layers F.Cu B.Cu) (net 18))
 (segment (start 207.01 128.19) (end 205.643 128.19) (width 0.26) (layer F.Cu) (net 18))
 (segment (start 204.875 128.19) (end 205.643 128.19) (width 0.26) (layer B.Cu) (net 18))
 (segment (start 203.11 126.425) (end 204.875 128.19) (width 0.26) (layer B.Cu) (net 18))
 (segment (start 203.11 125.98) (end 203.11 126.425) (width 0.26) (layer B.Cu) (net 18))
 (segment (start 202.22 125.98) (end 203.11 125.98) (width 0.26) (layer B.Cu) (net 18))
 (via (at 191.7271 143.7915) (size 0.889) (layers F.Cu B.Cu) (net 13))
 (segment (start 195.66 142.24) (end 195.66 142.2025) (width 0.5) (layer F.Cu) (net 13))
 (segment (start 196.22 138.18) (end 196.22 139.4303) (width 0.5) (layer B.Cu) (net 13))
 (segment (start 196.0883 139.4303) (end 196.22 139.4303) (width 0.5) (layer B.Cu) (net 13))
 (segment (start 191.7271 143.7915) (end 196.0883 139.4303) (width 0.5) (layer B.Cu) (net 13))
 (segment (start 194.071 143.7915) (end 191.7271 143.7915) (width 0.5) (layer F.Cu) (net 13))
 (segment (start 195.66 142.2025) (end 194.071 143.7915) (width 0.5) (layer F.Cu) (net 13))
 (segment (start 197.0228 140.8397) (end 195.66 142.2025) (width 0.5) (layer F.Cu) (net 13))
 (segment (start 203.28 140.8397) (end 197.0228 140.8397) (width 0.5) (layer F.Cu) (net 13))
 (segment (start 203.28 142.24) (end 203.28 140.8397) (width 0.5) (layer F.Cu) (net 13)))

